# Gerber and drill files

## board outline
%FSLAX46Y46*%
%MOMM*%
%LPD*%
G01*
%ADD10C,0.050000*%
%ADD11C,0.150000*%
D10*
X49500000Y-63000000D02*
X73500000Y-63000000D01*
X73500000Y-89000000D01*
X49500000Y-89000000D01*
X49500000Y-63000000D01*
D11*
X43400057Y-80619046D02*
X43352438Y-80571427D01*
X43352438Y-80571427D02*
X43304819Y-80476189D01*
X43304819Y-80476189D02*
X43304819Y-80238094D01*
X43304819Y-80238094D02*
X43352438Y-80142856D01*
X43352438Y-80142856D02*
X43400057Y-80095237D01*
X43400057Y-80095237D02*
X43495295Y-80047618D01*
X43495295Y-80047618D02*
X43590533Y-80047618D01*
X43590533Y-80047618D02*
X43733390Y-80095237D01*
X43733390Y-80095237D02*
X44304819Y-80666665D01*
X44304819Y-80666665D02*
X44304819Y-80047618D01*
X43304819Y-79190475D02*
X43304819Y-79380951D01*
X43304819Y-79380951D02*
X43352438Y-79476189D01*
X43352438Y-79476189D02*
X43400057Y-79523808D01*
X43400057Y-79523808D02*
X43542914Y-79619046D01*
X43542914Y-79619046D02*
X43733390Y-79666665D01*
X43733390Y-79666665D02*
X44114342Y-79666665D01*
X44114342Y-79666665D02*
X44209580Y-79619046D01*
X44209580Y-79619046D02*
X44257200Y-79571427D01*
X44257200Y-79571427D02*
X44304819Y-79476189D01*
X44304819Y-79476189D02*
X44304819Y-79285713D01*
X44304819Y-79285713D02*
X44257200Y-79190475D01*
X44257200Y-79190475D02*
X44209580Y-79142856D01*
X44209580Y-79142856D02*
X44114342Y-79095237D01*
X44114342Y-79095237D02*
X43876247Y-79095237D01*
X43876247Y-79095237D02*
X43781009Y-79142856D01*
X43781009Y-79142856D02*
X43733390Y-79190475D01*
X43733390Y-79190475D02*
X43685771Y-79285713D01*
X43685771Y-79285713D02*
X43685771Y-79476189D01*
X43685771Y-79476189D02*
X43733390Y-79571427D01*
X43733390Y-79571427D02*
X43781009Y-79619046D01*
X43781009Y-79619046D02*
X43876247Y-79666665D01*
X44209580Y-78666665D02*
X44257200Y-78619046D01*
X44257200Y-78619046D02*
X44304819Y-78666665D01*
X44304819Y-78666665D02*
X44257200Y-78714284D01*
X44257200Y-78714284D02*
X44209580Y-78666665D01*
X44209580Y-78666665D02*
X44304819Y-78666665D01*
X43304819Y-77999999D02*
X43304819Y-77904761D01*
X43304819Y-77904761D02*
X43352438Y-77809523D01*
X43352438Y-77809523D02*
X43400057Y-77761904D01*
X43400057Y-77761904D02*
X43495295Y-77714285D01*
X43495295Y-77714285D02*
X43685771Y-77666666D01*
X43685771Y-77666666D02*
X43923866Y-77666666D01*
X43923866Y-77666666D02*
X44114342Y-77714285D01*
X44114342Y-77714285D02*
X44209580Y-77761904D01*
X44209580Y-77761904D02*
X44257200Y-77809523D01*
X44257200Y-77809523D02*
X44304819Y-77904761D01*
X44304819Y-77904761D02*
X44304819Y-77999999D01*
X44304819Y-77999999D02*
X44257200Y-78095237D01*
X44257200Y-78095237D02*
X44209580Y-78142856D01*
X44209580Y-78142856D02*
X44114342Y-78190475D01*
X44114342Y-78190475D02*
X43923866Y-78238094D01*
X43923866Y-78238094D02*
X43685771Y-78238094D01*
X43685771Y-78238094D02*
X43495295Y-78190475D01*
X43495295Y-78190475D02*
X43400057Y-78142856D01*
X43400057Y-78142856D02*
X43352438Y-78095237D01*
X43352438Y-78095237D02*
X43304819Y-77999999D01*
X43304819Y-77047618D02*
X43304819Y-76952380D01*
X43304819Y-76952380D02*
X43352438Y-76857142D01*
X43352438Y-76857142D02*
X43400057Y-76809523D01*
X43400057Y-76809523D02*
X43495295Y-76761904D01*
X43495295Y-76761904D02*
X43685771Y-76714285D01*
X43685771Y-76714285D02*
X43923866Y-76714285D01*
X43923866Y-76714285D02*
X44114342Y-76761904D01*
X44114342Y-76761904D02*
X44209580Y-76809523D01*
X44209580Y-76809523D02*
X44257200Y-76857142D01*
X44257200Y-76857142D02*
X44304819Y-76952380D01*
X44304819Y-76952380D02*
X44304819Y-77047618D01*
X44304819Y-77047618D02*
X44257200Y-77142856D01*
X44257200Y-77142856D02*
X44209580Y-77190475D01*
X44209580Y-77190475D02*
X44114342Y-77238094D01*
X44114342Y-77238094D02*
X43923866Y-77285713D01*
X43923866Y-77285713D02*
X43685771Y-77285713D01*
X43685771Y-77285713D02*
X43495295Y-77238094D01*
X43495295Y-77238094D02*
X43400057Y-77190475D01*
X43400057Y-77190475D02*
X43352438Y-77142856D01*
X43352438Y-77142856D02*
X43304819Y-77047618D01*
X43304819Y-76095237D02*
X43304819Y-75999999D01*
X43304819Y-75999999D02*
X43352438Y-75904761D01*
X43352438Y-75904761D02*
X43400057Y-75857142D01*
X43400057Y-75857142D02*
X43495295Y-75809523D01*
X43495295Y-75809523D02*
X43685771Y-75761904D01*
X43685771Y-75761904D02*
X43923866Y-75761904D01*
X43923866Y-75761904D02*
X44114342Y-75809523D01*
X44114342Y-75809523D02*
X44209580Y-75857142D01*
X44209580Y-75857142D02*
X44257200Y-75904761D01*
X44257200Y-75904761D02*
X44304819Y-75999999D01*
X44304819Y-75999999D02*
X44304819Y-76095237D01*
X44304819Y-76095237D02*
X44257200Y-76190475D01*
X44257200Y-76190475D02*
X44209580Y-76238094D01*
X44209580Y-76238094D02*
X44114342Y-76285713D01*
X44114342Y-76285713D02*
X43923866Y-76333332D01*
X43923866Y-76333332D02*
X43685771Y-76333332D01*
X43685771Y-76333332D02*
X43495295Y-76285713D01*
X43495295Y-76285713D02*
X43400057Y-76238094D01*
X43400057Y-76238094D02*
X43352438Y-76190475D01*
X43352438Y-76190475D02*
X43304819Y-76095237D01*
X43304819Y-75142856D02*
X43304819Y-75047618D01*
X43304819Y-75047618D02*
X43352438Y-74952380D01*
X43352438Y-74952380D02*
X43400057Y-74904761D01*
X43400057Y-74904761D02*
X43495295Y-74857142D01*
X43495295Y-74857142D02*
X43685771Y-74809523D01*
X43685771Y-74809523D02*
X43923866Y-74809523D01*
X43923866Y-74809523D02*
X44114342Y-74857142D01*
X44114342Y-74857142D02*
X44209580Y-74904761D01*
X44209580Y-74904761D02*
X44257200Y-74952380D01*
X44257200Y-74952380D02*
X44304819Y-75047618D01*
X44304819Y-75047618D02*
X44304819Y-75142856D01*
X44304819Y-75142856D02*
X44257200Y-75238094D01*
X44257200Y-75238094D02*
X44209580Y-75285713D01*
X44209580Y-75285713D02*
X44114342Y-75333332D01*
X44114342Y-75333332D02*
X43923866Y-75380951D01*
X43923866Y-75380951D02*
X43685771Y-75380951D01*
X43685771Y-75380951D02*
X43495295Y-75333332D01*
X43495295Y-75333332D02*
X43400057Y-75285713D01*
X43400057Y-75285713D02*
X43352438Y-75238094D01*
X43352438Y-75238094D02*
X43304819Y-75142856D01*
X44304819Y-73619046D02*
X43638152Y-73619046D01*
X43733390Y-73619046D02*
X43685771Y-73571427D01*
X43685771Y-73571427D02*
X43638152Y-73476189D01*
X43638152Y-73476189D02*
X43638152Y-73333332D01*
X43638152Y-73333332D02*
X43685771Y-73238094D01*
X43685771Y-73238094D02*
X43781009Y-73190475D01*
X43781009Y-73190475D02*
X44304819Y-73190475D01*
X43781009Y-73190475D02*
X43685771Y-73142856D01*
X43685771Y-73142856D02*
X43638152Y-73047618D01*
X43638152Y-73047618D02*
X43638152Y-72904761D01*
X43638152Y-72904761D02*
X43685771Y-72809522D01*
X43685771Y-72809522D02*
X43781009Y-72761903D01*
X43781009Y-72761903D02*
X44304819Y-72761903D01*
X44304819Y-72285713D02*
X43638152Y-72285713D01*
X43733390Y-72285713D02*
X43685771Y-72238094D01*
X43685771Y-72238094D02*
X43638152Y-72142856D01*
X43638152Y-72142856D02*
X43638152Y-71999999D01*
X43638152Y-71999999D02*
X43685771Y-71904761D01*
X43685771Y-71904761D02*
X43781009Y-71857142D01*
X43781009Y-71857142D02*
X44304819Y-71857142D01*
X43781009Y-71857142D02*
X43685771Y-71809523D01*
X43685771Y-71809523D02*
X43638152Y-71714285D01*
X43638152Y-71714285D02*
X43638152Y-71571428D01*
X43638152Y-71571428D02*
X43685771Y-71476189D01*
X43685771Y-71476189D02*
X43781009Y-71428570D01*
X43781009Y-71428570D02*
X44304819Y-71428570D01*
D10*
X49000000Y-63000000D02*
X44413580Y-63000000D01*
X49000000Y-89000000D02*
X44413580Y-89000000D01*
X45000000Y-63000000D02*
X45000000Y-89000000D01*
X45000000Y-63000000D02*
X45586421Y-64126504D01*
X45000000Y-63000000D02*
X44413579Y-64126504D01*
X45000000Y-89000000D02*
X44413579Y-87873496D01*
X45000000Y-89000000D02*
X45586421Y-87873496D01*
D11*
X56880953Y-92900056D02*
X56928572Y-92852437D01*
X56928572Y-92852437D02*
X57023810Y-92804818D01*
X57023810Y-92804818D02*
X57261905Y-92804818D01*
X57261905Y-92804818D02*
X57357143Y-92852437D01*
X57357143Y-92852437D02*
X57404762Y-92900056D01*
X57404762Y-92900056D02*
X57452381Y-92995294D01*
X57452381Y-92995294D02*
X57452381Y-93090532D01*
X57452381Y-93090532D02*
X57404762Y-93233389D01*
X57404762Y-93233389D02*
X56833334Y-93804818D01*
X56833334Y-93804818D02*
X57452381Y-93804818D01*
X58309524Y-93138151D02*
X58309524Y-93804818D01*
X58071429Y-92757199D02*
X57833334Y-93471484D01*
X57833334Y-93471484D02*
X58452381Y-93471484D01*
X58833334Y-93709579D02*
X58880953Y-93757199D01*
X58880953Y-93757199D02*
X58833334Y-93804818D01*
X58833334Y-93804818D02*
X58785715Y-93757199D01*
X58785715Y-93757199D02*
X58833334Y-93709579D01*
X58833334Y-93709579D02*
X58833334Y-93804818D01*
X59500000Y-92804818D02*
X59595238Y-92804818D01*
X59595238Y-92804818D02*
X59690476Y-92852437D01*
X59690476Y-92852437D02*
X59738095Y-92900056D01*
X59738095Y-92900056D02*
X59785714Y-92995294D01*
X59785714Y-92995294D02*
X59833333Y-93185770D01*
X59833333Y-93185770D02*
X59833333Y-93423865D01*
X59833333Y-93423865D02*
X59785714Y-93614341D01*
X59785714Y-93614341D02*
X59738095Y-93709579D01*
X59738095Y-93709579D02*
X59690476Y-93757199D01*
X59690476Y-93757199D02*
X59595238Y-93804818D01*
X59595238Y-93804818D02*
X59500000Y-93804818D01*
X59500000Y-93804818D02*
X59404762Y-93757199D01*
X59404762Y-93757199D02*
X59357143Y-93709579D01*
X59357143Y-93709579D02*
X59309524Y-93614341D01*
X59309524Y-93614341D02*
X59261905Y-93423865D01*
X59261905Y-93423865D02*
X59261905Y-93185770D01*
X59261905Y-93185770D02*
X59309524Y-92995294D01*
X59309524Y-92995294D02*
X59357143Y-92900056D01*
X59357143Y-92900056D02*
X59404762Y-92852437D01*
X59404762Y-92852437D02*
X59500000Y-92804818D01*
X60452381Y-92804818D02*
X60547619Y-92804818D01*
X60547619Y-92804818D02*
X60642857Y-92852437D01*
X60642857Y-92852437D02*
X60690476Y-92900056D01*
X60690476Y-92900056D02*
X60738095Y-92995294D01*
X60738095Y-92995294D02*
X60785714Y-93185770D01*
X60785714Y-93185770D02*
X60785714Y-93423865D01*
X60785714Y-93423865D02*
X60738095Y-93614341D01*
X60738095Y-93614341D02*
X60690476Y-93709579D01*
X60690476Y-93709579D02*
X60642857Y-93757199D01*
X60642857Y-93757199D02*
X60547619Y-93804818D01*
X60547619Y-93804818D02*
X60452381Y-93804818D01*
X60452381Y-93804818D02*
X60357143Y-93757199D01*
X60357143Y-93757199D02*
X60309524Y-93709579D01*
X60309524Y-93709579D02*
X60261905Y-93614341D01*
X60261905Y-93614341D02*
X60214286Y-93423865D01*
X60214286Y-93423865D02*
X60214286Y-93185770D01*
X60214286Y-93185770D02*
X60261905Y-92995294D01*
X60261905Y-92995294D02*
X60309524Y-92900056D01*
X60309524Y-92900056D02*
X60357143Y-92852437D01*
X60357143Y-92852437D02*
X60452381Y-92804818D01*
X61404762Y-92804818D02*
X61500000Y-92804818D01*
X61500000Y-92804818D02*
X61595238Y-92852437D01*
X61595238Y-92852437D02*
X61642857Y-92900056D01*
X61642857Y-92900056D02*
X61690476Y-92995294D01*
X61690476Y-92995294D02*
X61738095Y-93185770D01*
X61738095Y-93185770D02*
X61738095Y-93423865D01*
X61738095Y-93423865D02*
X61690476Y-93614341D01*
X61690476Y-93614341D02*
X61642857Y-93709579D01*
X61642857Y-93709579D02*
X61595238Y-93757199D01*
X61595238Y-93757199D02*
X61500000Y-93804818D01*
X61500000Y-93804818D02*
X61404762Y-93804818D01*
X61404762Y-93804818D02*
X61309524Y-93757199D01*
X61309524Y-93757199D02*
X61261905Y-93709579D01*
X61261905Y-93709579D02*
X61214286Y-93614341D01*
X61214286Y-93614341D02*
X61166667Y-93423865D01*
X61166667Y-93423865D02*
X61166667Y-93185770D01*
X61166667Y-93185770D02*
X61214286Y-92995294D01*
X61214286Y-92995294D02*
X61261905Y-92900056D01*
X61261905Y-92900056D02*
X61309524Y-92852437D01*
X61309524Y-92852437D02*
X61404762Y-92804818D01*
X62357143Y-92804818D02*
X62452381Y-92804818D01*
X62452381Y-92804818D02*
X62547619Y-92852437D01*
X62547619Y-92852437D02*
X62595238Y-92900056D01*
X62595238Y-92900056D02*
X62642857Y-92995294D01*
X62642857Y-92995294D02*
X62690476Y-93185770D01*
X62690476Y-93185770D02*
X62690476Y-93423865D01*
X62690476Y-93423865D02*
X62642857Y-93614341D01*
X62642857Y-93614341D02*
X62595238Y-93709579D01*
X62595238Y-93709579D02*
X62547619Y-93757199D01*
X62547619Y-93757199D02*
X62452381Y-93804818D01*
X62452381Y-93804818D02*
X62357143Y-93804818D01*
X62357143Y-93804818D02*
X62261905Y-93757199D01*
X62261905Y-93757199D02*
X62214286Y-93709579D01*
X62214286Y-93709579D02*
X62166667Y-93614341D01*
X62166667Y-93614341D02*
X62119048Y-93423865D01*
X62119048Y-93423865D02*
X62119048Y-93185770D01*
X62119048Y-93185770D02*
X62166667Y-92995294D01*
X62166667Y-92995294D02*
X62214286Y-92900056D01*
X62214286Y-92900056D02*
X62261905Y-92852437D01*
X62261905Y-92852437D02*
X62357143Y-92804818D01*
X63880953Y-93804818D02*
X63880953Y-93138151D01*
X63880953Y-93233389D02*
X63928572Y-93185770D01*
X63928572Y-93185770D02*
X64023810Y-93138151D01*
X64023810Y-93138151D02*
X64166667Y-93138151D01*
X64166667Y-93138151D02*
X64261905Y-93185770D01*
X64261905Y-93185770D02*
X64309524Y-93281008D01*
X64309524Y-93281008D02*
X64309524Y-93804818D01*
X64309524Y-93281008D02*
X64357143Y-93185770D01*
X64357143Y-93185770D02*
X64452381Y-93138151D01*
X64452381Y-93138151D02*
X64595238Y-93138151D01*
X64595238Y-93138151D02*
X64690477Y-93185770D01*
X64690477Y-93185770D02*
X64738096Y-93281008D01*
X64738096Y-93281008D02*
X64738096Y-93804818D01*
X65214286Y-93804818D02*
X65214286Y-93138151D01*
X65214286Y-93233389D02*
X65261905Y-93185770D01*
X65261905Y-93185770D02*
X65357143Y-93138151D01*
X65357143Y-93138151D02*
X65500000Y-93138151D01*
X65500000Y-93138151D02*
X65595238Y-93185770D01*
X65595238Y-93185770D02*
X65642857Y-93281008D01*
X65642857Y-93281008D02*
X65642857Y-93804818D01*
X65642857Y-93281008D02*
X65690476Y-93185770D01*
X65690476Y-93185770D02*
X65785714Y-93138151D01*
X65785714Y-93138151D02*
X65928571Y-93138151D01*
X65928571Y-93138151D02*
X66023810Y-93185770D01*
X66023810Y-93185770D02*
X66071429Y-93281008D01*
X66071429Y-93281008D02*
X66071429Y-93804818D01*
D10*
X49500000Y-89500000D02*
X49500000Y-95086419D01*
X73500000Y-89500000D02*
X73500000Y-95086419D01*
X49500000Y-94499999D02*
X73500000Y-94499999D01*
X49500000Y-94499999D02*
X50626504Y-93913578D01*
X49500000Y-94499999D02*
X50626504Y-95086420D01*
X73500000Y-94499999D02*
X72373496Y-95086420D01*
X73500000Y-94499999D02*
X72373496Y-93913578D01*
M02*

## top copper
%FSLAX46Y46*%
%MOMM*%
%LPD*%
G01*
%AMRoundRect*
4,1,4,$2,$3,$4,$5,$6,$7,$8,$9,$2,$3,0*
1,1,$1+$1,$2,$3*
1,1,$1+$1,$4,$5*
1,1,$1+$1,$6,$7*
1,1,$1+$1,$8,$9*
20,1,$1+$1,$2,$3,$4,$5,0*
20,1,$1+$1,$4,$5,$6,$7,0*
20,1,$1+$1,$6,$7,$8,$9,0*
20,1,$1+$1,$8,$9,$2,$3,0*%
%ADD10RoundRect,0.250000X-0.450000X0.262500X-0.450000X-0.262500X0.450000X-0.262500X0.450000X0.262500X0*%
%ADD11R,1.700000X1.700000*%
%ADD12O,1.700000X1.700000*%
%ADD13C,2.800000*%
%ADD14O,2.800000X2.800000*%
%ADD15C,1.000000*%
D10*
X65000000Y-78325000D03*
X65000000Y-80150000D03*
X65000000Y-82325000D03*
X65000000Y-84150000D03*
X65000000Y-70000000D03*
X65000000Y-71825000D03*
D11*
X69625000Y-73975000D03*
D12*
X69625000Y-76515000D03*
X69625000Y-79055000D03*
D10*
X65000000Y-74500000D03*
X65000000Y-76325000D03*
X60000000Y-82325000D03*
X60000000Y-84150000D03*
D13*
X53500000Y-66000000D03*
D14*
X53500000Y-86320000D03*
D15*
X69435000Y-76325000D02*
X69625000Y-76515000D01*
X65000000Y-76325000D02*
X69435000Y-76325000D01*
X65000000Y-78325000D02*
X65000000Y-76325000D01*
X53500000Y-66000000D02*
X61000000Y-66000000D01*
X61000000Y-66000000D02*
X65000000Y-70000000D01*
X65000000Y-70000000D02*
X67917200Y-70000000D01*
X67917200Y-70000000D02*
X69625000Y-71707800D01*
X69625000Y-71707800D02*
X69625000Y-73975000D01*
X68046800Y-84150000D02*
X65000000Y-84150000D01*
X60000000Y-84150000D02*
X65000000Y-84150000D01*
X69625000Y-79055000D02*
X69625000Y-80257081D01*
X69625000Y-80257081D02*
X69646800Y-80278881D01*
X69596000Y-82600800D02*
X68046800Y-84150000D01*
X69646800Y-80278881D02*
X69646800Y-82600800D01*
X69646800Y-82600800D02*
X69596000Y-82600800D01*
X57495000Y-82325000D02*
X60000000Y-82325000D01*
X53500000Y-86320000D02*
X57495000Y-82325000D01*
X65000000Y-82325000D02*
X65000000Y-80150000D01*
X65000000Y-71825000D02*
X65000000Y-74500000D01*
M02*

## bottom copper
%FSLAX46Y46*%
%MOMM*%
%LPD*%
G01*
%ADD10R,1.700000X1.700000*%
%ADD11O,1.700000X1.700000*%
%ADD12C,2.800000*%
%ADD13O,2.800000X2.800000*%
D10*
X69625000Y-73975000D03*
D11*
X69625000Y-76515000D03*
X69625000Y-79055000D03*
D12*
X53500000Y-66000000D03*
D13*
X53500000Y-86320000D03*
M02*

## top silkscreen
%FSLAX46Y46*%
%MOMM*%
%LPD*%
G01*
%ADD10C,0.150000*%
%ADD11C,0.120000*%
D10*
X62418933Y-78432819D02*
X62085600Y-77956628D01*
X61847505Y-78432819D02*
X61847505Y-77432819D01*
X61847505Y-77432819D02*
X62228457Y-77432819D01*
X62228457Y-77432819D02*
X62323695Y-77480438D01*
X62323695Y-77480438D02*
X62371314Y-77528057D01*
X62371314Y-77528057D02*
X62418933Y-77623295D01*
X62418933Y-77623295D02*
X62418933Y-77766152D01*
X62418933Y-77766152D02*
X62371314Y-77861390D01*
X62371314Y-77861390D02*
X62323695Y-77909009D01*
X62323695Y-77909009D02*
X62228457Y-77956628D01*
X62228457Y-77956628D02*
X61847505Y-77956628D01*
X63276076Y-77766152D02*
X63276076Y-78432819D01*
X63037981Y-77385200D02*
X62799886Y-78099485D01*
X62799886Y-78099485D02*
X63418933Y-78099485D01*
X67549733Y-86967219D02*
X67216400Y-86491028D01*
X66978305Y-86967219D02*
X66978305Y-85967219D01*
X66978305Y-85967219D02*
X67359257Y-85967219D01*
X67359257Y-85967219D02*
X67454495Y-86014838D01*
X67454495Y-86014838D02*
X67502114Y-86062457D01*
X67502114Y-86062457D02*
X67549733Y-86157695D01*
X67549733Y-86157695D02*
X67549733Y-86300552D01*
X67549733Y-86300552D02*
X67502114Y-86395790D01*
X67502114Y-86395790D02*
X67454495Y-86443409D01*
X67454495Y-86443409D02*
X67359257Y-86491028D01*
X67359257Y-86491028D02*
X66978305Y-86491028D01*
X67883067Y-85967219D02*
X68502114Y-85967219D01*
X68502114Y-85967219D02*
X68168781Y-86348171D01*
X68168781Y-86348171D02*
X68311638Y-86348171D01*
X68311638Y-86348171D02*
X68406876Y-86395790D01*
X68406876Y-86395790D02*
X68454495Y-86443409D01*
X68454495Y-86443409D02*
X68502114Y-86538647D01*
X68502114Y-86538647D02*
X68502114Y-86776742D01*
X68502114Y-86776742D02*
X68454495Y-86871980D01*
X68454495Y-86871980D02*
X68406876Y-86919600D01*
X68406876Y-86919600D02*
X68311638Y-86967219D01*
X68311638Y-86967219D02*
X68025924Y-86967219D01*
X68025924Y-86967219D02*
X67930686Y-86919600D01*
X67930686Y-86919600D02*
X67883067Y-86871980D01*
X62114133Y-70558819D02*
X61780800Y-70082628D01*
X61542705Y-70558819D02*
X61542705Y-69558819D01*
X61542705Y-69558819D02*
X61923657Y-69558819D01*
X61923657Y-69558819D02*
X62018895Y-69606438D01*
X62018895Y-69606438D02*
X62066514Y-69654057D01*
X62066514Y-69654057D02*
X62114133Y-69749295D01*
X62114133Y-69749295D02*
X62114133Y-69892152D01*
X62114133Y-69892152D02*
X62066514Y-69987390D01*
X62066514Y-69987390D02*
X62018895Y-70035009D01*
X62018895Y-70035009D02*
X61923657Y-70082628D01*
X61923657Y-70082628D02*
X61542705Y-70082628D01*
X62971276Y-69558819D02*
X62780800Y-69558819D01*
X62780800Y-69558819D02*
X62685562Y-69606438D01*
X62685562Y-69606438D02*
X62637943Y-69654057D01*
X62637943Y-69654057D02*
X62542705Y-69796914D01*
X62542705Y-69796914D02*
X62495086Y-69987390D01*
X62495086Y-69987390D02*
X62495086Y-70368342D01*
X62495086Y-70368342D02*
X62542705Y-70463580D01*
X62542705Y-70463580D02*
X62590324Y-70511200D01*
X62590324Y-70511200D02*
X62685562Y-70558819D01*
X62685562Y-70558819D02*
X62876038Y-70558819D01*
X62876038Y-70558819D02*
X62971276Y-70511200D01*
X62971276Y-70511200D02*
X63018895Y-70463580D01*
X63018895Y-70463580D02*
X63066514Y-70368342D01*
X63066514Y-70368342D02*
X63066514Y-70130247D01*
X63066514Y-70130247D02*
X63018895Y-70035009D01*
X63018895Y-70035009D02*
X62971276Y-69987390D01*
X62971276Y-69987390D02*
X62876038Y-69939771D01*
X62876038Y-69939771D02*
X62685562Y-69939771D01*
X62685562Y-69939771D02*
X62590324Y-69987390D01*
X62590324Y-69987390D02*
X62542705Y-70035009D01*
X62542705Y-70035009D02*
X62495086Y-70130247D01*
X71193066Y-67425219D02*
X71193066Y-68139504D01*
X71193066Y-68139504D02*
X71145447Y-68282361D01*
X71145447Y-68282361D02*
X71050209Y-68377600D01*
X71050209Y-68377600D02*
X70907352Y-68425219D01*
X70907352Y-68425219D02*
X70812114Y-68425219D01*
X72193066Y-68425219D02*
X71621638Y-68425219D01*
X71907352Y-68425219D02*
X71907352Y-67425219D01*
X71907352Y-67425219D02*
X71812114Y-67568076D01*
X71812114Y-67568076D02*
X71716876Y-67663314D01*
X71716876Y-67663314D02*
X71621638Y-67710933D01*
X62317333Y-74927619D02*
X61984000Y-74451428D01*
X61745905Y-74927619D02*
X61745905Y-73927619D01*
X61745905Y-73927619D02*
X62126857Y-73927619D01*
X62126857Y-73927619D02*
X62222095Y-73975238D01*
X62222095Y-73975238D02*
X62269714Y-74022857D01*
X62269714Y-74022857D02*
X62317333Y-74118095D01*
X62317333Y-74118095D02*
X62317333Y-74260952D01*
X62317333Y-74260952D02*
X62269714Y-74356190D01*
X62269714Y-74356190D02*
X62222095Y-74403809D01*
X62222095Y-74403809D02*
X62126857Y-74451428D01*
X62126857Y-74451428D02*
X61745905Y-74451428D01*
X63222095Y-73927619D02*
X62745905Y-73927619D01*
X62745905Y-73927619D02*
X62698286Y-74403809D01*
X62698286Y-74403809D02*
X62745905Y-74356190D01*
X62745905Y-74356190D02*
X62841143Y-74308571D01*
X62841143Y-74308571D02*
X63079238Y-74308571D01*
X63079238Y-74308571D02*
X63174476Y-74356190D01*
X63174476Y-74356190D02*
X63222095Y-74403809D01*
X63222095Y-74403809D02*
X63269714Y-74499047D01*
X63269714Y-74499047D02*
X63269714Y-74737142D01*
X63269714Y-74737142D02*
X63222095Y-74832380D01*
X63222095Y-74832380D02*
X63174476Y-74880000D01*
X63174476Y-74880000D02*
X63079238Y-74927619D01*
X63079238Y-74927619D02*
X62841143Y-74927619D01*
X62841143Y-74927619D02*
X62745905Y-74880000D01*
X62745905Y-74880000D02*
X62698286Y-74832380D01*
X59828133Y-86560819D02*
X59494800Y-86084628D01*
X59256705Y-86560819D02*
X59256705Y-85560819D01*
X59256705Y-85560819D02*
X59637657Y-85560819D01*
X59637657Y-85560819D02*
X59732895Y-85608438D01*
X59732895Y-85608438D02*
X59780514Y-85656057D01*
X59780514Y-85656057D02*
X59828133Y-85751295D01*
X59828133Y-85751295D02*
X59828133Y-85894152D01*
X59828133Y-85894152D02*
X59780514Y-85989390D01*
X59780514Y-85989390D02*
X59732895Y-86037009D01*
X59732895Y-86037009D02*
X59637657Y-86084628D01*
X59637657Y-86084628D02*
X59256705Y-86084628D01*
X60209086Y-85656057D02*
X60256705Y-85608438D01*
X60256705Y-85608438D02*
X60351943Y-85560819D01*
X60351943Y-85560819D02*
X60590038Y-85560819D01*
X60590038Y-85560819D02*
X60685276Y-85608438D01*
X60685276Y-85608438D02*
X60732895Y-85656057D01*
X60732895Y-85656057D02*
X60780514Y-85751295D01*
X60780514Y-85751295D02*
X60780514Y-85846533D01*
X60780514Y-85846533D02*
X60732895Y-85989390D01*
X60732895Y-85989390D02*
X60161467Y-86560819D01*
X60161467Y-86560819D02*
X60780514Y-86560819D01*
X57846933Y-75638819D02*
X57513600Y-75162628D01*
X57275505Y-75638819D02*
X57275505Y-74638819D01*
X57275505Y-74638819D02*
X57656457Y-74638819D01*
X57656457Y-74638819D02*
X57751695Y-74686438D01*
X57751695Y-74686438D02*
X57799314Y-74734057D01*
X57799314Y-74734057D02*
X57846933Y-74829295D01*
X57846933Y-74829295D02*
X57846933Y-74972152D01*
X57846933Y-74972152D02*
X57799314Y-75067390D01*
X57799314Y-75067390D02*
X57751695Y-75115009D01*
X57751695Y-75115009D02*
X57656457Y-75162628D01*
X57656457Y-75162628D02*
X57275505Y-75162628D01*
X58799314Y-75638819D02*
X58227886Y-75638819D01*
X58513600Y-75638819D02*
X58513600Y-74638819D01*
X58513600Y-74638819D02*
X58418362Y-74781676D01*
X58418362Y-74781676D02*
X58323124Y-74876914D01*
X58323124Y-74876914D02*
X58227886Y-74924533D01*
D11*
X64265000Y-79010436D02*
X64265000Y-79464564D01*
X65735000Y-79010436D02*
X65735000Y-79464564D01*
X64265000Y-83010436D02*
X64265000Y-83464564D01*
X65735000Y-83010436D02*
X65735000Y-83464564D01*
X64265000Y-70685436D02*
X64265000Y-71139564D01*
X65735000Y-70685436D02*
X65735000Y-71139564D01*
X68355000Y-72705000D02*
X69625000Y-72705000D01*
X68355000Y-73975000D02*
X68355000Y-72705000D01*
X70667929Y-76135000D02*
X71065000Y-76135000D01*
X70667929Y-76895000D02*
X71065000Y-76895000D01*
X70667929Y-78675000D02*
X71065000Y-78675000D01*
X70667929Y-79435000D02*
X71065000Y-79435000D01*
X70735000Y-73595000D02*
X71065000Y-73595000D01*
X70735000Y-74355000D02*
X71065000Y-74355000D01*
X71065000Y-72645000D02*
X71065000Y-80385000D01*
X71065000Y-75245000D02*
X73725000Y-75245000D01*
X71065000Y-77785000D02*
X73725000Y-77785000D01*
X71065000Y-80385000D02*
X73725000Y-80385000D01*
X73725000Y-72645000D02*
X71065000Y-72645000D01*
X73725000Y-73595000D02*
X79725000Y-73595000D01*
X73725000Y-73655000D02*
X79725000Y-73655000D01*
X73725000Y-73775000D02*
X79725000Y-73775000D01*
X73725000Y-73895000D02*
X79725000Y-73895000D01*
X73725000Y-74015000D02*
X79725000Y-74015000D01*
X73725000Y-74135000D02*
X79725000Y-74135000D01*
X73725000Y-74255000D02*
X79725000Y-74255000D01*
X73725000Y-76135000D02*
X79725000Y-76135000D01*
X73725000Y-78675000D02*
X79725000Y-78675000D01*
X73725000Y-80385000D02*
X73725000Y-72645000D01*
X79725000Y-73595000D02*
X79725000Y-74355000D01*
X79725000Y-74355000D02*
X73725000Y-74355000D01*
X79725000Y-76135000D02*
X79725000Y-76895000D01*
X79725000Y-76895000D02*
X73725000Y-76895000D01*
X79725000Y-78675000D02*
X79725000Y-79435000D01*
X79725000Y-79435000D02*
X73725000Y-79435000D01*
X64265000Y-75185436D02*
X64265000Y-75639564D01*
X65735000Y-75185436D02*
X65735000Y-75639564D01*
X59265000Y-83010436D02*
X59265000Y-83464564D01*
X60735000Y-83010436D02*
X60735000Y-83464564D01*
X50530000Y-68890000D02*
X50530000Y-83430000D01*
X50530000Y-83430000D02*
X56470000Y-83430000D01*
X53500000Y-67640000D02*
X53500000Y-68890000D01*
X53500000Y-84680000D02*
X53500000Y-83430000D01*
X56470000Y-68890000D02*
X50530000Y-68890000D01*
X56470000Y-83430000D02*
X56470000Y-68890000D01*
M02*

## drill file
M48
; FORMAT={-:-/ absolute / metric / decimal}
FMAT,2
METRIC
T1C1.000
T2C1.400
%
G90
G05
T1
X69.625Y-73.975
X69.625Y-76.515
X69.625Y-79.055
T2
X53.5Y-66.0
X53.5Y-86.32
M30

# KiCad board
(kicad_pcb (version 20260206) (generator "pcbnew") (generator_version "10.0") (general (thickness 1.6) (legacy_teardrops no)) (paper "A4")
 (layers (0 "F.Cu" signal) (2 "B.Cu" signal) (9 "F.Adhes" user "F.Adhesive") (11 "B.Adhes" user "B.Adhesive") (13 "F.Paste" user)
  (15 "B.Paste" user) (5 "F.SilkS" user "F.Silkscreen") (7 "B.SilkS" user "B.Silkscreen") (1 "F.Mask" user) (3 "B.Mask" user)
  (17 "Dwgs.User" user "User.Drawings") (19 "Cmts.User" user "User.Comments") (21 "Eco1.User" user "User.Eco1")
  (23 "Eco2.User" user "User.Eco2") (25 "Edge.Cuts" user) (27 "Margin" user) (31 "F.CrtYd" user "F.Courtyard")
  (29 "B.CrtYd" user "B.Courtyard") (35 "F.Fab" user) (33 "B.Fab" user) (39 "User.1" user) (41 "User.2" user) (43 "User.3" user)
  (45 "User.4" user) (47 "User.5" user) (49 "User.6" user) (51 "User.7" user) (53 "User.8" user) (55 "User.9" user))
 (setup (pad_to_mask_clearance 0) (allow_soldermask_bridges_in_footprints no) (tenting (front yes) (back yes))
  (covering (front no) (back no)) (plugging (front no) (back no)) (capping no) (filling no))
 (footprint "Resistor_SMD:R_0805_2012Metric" (layer "F.Cu") (at 65 79.2375 -90)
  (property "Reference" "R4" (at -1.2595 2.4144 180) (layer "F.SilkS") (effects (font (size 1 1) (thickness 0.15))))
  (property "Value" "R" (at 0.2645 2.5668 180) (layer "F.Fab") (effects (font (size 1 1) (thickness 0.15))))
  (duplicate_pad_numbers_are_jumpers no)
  (fp_line (start -0.227064 0.735) (end 0.227064 0.735) (stroke (width 0.12) (type solid)) (layer "F.SilkS"))
  (fp_line (start -0.227064 -0.735) (end 0.227064 -0.735) (stroke (width 0.12) (type solid)) (layer "F.SilkS"))
  (pad "1" smd roundrect (at -0.9125 0 270) (size 1.025 1.4) (layers "F.Cu" "F.Mask" "F.Paste") (roundrect_rratio 0.243902) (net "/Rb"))
  (pad "2" smd roundrect (at 0.9125 0 270) (size 1.025 1.4) (layers "F.Cu" "F.Mask" "F.Paste") (roundrect_rratio 0.243902)
   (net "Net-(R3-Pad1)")))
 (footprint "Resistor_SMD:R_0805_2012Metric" (layer "F.Cu") (at 65 83.2375 -90)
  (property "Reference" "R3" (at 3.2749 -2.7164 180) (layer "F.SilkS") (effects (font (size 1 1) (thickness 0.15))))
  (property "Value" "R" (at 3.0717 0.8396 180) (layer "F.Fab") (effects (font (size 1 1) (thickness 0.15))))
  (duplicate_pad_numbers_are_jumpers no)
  (fp_line (start -0.227064 0.735) (end 0.227064 0.735) (stroke (width 0.12) (type solid)) (layer "F.SilkS"))
  (fp_line (start -0.227064 -0.735) (end 0.227064 -0.735) (stroke (width 0.12) (type solid)) (layer "F.SilkS"))
  (pad "1" smd roundrect (at -0.9125 0 270) (size 1.025 1.4) (layers "F.Cu" "F.Mask" "F.Paste") (roundrect_rratio 0.243902)
   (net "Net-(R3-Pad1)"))
  (pad "2" smd roundrect (at 0.9125 0 270) (size 1.025 1.4) (layers "F.Cu" "F.Mask" "F.Paste") (roundrect_rratio 0.243902) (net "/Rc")))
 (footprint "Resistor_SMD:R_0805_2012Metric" (layer "F.Cu") (at 65 70.9125 -90)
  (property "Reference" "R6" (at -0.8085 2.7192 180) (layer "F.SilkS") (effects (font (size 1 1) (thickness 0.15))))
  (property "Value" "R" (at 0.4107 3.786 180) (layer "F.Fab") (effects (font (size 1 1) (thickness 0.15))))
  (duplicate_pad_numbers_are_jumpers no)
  (fp_line (start -0.227064 0.735) (end 0.227064 0.735) (stroke (width 0.12) (type solid)) (layer "F.SilkS"))
  (fp_line (start -0.227064 -0.735) (end 0.227064 -0.735) (stroke (width 0.12) (type solid)) (layer "F.SilkS"))
  (pad "1" smd roundrect (at -0.9125 0 270) (size 1.025 1.4) (layers "F.Cu" "F.Mask" "F.Paste") (roundrect_rratio 0.243902) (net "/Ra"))
  (pad "2" smd roundrect (at 0.9125 0 270) (size 1.025 1.4) (layers "F.Cu" "F.Mask" "F.Paste") (roundrect_rratio 0.243902)
   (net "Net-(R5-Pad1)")))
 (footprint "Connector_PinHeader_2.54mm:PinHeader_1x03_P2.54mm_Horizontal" (layer "F.Cu") (at 69.625 73.975)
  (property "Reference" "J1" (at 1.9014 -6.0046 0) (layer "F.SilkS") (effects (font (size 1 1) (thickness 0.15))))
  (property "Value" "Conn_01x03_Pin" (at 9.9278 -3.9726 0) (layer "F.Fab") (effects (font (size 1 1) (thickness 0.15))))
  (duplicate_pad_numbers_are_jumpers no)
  (fp_line (start -1.27 -1.27) (end 0 -1.27) (stroke (width 0.12) (type solid)) (layer "F.SilkS"))
  (fp_line (start -1.27 0) (end -1.27 -1.27) (stroke (width 0.12) (type solid)) (layer "F.SilkS"))
  (fp_line (start 1.042929 2.16) (end 1.44 2.16) (stroke (width 0.12) (type solid)) (layer "F.SilkS"))
  (fp_line (start 1.042929 2.92) (end 1.44 2.92) (stroke (width 0.12) (type solid)) (layer "F.SilkS"))
  (fp_line (start 1.042929 4.7) (end 1.44 4.7) (stroke (width 0.12) (type solid)) (layer "F.SilkS"))
  (fp_line (start 1.042929 5.46) (end 1.44 5.46) (stroke (width 0.12) (type solid)) (layer "F.SilkS"))
  (fp_line (start 1.11 -0.38) (end 1.44 -0.38) (stroke (width 0.12) (type solid)) (layer "F.SilkS"))
  (fp_line (start 1.11 0.38) (end 1.44 0.38) (stroke (width 0.12) (type solid)) (layer "F.SilkS"))
  (fp_line (start 1.44 -1.33) (end 1.44 6.41) (stroke (width 0.12) (type solid)) (layer "F.SilkS"))
  (fp_line (start 1.44 1.27) (end 4.1 1.27) (stroke (width 0.12) (type solid)) (layer "F.SilkS"))
  (fp_line (start 1.44 3.81) (end 4.1 3.81) (stroke (width 0.12) (type solid)) (layer "F.SilkS"))
  (fp_line (start 1.44 6.41) (end 4.1 6.41) (stroke (width 0.12) (type solid)) (layer "F.SilkS"))
  (fp_line (start 4.1 -1.33) (end 1.44 -1.33) (stroke (width 0.12) (type solid)) (layer "F.SilkS"))
  (fp_line (start 4.1 -0.38) (end 10.1 -0.38) (stroke (width 0.12) (type solid)) (layer "F.SilkS"))
  (fp_line (start 4.1 -0.32) (end 10.1 -0.32) (stroke (width 0.12) (type solid)) (layer "F.SilkS"))
  (fp_line (start 4.1 -0.2) (end 10.1 -0.2) (stroke (width 0.12) (type solid)) (layer "F.SilkS"))
  (fp_line (start 4.1 -0.08) (end 10.1 -0.08) (stroke (width 0.12) (type solid)) (layer "F.SilkS"))
  (fp_line (start 4.1 0.04) (end 10.1 0.04) (stroke (width 0.12) (type solid)) (layer "F.SilkS"))
  (fp_line (start 4.1 0.16) (end 10.1 0.16) (stroke (width 0.12) (type solid)) (layer "F.SilkS"))
  (fp_line (start 4.1 0.28) (end 10.1 0.28) (stroke (width 0.12) (type solid)) (layer "F.SilkS"))
  (fp_line (start 4.1 2.16) (end 10.1 2.16) (stroke (width 0.12) (type solid)) (layer "F.SilkS"))
  (fp_line (start 4.1 4.7) (end 10.1 4.7) (stroke (width 0.12) (type solid)) (layer "F.SilkS"))
  (fp_line (start 4.1 6.41) (end 4.1 -1.33) (stroke (width 0.12) (type solid)) (layer "F.SilkS"))
  (fp_line (start 10.1 -0.38) (end 10.1 0.38) (stroke (width 0.12) (type solid)) (layer "F.SilkS"))
  (fp_line (start 10.1 0.38) (end 4.1 0.38) (stroke (width 0.12) (type solid)) (layer "F.SilkS"))
  (fp_line (start 10.1 2.16) (end 10.1 2.92) (stroke (width 0.12) (type solid)) (layer "F.SilkS"))
  (fp_line (start 10.1 2.92) (end 4.1 2.92) (stroke (width 0.12) (type solid)) (layer "F.SilkS"))
  (fp_line (start 10.1 4.7) (end 10.1 5.46) (stroke (width 0.12) (type solid)) (layer "F.SilkS"))
  (fp_line (start 10.1 5.46) (end 4.1 5.46) (stroke (width 0.12) (type solid)) (layer "F.SilkS"))
  (pad "1" thru_hole rect (at 0 0) (size 1.7 1.7) (drill 1) (layers "*.Cu" "*.Mask") (remove_unused_layers no) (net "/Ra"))
  (pad "2" thru_hole oval (at 0 2.54) (size 1.7 1.7) (drill 1) (layers "*.Cu" "*.Mask") (remove_unused_layers no) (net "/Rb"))
  (pad "3" thru_hole oval (at 0 5.08) (size 1.7 1.7) (drill 1) (layers "*.Cu" "*.Mask") (remove_unused_layers no) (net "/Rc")))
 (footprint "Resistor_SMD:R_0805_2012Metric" (layer "F.Cu") (at 65 75.4125 -90)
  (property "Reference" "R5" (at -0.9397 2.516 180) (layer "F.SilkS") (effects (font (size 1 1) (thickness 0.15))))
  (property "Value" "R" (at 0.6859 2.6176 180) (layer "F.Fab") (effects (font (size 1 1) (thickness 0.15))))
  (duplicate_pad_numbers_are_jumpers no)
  (fp_line (start -0.227064 0.735) (end 0.227064 0.735) (stroke (width 0.12) (type solid)) (layer "F.SilkS"))
  (fp_line (start -0.227064 -0.735) (end 0.227064 -0.735) (stroke (width 0.12) (type solid)) (layer "F.SilkS"))
  (pad "1" smd roundrect (at -0.9125 0 270) (size 1.025 1.4) (layers "F.Cu" "F.Mask" "F.Paste") (roundrect_rratio 0.243902)
   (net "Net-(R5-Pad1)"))
  (pad "2" smd roundrect (at 0.9125 0 270) (size 1.025 1.4) (layers "F.Cu" "F.Mask" "F.Paste") (roundrect_rratio 0.243902) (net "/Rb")))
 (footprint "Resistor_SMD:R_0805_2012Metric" (layer "F.Cu") (at 60 83.2375 -90)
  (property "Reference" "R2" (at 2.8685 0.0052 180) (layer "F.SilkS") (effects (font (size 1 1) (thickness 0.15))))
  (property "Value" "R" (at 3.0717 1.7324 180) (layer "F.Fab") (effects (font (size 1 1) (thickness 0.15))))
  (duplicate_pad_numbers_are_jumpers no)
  (fp_line (start -0.227064 0.735) (end 0.227064 0.735) (stroke (width 0.12) (type solid)) (layer "F.SilkS"))
  (fp_line (start -0.227064 -0.735) (end 0.227064 -0.735) (stroke (width 0.12) (type solid)) (layer "F.SilkS"))
  (pad "1" smd roundrect (at -0.9125 0 270) (size 1.025 1.4) (layers "F.Cu" "F.Mask" "F.Paste") (roundrect_rratio 0.243902)
   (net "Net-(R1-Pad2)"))
  (pad "2" smd roundrect (at 0.9125 0 270) (size 1.025 1.4) (layers "F.Cu" "F.Mask" "F.Paste") (roundrect_rratio 0.243902) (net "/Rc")))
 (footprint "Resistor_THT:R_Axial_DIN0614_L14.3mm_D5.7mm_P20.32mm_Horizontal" (layer "F.Cu") (at 53.5 66 -90)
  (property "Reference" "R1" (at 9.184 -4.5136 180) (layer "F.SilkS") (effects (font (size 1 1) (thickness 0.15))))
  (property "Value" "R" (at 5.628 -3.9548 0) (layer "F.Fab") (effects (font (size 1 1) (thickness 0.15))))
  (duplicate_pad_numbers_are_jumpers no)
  (fp_line (start 2.89 2.97) (end 17.43 2.97) (stroke (width 0.12) (type solid)) (layer "F.SilkS"))
  (fp_line (start 17.43 2.97) (end 17.43 -2.97) (stroke (width 0.12) (type solid)) (layer "F.SilkS"))
  (fp_line (start 1.64 0) (end 2.89 0) (stroke (width 0.12) (type solid)) (layer "F.SilkS"))
  (fp_line (start 18.68 0) (end 17.43 0) (stroke (width 0.12) (type solid)) (layer "F.SilkS"))
  (fp_line (start 2.89 -2.97) (end 2.89 2.97) (stroke (width 0.12) (type solid)) (layer "F.SilkS"))
  (fp_line (start 17.43 -2.97) (end 2.89 -2.97) (stroke (width 0.12) (type solid)) (layer "F.SilkS"))
  (pad "1" thru_hole circle (at 0 0 270) (size 2.8 2.8) (drill 1.4) (layers "*.Cu" "*.Mask") (remove_unused_layers no) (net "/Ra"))
  (pad "2" thru_hole oval (at 20.32 0 270) (size 2.8 2.8) (drill 1.4) (layers "*.Cu" "*.Mask") (remove_unused_layers no)
   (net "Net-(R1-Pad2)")))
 (gr_rect (start 49.5 63) (end 73.5 89) (stroke (width 0.05) (type default)) (fill no) (layer "Edge.Cuts"))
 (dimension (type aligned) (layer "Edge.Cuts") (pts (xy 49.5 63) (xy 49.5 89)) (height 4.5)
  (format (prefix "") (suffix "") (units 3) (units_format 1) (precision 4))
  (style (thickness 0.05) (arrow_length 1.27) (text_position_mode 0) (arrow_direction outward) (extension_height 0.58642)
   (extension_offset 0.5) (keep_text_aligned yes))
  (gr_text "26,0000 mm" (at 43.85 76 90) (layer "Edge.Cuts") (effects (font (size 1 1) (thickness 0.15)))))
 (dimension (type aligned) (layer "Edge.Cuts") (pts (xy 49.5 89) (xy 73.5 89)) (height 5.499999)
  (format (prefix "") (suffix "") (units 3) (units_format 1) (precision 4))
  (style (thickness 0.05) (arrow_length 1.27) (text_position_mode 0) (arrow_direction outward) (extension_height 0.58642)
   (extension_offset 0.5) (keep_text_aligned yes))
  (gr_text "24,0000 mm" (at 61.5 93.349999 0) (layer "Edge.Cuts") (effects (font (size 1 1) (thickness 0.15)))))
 (segment (start 69.435 76.325) (end 69.625 76.515) (width 1) (layer "F.Cu") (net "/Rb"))
 (segment (start 65 76.325) (end 69.435 76.325) (width 1) (layer "F.Cu") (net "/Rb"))
 (segment (start 65 78.325) (end 65 76.325) (width 1) (layer "F.Cu") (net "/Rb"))
 (segment (start 53.5 66) (end 61 66) (width 1) (layer "F.Cu") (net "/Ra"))
 (segment (start 61 66) (end 65 70) (width 1) (layer "F.Cu") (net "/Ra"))
 (segment (start 65 70) (end 67.9172 70) (width 1) (layer "F.Cu") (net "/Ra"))
 (segment (start 67.9172 70) (end 69.625 71.7078) (width 1) (layer "F.Cu") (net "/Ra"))
 (segment (start 69.625 71.7078) (end 69.625 73.975) (width 1) (layer "F.Cu") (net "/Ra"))
 (segment (start 68.0468 84.15) (end 65 84.15) (width 1) (layer "F.Cu") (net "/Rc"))
 (segment (start 60 84.15) (end 65 84.15) (width 1) (layer "F.Cu") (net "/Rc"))
 (segment (start 69.625 79.055) (end 69.625 80.257081) (width 1) (layer "F.Cu") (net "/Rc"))
 (segment (start 69.625 80.257081) (end 69.6468 80.278881) (width 1) (layer "F.Cu") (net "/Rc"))
 (segment (start 69.596 82.6008) (end 68.0468 84.15) (width 1) (layer "F.Cu") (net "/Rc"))
 (segment (start 69.6468 80.278881) (end 69.6468 82.6008) (width 1) (layer "F.Cu") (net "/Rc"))
 (segment (start 69.6468 82.6008) (end 69.596 82.6008) (width 1) (layer "F.Cu") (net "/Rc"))
 (segment (start 57.495 82.325) (end 60 82.325) (width 1) (layer "F.Cu") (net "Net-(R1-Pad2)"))
 (segment (start 53.5 86.32) (end 57.495 82.325) (width 1) (layer "F.Cu") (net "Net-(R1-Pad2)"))
 (segment (start 65 82.325) (end 65 80.15) (width 1) (layer "F.Cu") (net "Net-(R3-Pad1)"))
 (segment (start 65 71.825) (end 65 74.5) (width 1) (layer "F.Cu") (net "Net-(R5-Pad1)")))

